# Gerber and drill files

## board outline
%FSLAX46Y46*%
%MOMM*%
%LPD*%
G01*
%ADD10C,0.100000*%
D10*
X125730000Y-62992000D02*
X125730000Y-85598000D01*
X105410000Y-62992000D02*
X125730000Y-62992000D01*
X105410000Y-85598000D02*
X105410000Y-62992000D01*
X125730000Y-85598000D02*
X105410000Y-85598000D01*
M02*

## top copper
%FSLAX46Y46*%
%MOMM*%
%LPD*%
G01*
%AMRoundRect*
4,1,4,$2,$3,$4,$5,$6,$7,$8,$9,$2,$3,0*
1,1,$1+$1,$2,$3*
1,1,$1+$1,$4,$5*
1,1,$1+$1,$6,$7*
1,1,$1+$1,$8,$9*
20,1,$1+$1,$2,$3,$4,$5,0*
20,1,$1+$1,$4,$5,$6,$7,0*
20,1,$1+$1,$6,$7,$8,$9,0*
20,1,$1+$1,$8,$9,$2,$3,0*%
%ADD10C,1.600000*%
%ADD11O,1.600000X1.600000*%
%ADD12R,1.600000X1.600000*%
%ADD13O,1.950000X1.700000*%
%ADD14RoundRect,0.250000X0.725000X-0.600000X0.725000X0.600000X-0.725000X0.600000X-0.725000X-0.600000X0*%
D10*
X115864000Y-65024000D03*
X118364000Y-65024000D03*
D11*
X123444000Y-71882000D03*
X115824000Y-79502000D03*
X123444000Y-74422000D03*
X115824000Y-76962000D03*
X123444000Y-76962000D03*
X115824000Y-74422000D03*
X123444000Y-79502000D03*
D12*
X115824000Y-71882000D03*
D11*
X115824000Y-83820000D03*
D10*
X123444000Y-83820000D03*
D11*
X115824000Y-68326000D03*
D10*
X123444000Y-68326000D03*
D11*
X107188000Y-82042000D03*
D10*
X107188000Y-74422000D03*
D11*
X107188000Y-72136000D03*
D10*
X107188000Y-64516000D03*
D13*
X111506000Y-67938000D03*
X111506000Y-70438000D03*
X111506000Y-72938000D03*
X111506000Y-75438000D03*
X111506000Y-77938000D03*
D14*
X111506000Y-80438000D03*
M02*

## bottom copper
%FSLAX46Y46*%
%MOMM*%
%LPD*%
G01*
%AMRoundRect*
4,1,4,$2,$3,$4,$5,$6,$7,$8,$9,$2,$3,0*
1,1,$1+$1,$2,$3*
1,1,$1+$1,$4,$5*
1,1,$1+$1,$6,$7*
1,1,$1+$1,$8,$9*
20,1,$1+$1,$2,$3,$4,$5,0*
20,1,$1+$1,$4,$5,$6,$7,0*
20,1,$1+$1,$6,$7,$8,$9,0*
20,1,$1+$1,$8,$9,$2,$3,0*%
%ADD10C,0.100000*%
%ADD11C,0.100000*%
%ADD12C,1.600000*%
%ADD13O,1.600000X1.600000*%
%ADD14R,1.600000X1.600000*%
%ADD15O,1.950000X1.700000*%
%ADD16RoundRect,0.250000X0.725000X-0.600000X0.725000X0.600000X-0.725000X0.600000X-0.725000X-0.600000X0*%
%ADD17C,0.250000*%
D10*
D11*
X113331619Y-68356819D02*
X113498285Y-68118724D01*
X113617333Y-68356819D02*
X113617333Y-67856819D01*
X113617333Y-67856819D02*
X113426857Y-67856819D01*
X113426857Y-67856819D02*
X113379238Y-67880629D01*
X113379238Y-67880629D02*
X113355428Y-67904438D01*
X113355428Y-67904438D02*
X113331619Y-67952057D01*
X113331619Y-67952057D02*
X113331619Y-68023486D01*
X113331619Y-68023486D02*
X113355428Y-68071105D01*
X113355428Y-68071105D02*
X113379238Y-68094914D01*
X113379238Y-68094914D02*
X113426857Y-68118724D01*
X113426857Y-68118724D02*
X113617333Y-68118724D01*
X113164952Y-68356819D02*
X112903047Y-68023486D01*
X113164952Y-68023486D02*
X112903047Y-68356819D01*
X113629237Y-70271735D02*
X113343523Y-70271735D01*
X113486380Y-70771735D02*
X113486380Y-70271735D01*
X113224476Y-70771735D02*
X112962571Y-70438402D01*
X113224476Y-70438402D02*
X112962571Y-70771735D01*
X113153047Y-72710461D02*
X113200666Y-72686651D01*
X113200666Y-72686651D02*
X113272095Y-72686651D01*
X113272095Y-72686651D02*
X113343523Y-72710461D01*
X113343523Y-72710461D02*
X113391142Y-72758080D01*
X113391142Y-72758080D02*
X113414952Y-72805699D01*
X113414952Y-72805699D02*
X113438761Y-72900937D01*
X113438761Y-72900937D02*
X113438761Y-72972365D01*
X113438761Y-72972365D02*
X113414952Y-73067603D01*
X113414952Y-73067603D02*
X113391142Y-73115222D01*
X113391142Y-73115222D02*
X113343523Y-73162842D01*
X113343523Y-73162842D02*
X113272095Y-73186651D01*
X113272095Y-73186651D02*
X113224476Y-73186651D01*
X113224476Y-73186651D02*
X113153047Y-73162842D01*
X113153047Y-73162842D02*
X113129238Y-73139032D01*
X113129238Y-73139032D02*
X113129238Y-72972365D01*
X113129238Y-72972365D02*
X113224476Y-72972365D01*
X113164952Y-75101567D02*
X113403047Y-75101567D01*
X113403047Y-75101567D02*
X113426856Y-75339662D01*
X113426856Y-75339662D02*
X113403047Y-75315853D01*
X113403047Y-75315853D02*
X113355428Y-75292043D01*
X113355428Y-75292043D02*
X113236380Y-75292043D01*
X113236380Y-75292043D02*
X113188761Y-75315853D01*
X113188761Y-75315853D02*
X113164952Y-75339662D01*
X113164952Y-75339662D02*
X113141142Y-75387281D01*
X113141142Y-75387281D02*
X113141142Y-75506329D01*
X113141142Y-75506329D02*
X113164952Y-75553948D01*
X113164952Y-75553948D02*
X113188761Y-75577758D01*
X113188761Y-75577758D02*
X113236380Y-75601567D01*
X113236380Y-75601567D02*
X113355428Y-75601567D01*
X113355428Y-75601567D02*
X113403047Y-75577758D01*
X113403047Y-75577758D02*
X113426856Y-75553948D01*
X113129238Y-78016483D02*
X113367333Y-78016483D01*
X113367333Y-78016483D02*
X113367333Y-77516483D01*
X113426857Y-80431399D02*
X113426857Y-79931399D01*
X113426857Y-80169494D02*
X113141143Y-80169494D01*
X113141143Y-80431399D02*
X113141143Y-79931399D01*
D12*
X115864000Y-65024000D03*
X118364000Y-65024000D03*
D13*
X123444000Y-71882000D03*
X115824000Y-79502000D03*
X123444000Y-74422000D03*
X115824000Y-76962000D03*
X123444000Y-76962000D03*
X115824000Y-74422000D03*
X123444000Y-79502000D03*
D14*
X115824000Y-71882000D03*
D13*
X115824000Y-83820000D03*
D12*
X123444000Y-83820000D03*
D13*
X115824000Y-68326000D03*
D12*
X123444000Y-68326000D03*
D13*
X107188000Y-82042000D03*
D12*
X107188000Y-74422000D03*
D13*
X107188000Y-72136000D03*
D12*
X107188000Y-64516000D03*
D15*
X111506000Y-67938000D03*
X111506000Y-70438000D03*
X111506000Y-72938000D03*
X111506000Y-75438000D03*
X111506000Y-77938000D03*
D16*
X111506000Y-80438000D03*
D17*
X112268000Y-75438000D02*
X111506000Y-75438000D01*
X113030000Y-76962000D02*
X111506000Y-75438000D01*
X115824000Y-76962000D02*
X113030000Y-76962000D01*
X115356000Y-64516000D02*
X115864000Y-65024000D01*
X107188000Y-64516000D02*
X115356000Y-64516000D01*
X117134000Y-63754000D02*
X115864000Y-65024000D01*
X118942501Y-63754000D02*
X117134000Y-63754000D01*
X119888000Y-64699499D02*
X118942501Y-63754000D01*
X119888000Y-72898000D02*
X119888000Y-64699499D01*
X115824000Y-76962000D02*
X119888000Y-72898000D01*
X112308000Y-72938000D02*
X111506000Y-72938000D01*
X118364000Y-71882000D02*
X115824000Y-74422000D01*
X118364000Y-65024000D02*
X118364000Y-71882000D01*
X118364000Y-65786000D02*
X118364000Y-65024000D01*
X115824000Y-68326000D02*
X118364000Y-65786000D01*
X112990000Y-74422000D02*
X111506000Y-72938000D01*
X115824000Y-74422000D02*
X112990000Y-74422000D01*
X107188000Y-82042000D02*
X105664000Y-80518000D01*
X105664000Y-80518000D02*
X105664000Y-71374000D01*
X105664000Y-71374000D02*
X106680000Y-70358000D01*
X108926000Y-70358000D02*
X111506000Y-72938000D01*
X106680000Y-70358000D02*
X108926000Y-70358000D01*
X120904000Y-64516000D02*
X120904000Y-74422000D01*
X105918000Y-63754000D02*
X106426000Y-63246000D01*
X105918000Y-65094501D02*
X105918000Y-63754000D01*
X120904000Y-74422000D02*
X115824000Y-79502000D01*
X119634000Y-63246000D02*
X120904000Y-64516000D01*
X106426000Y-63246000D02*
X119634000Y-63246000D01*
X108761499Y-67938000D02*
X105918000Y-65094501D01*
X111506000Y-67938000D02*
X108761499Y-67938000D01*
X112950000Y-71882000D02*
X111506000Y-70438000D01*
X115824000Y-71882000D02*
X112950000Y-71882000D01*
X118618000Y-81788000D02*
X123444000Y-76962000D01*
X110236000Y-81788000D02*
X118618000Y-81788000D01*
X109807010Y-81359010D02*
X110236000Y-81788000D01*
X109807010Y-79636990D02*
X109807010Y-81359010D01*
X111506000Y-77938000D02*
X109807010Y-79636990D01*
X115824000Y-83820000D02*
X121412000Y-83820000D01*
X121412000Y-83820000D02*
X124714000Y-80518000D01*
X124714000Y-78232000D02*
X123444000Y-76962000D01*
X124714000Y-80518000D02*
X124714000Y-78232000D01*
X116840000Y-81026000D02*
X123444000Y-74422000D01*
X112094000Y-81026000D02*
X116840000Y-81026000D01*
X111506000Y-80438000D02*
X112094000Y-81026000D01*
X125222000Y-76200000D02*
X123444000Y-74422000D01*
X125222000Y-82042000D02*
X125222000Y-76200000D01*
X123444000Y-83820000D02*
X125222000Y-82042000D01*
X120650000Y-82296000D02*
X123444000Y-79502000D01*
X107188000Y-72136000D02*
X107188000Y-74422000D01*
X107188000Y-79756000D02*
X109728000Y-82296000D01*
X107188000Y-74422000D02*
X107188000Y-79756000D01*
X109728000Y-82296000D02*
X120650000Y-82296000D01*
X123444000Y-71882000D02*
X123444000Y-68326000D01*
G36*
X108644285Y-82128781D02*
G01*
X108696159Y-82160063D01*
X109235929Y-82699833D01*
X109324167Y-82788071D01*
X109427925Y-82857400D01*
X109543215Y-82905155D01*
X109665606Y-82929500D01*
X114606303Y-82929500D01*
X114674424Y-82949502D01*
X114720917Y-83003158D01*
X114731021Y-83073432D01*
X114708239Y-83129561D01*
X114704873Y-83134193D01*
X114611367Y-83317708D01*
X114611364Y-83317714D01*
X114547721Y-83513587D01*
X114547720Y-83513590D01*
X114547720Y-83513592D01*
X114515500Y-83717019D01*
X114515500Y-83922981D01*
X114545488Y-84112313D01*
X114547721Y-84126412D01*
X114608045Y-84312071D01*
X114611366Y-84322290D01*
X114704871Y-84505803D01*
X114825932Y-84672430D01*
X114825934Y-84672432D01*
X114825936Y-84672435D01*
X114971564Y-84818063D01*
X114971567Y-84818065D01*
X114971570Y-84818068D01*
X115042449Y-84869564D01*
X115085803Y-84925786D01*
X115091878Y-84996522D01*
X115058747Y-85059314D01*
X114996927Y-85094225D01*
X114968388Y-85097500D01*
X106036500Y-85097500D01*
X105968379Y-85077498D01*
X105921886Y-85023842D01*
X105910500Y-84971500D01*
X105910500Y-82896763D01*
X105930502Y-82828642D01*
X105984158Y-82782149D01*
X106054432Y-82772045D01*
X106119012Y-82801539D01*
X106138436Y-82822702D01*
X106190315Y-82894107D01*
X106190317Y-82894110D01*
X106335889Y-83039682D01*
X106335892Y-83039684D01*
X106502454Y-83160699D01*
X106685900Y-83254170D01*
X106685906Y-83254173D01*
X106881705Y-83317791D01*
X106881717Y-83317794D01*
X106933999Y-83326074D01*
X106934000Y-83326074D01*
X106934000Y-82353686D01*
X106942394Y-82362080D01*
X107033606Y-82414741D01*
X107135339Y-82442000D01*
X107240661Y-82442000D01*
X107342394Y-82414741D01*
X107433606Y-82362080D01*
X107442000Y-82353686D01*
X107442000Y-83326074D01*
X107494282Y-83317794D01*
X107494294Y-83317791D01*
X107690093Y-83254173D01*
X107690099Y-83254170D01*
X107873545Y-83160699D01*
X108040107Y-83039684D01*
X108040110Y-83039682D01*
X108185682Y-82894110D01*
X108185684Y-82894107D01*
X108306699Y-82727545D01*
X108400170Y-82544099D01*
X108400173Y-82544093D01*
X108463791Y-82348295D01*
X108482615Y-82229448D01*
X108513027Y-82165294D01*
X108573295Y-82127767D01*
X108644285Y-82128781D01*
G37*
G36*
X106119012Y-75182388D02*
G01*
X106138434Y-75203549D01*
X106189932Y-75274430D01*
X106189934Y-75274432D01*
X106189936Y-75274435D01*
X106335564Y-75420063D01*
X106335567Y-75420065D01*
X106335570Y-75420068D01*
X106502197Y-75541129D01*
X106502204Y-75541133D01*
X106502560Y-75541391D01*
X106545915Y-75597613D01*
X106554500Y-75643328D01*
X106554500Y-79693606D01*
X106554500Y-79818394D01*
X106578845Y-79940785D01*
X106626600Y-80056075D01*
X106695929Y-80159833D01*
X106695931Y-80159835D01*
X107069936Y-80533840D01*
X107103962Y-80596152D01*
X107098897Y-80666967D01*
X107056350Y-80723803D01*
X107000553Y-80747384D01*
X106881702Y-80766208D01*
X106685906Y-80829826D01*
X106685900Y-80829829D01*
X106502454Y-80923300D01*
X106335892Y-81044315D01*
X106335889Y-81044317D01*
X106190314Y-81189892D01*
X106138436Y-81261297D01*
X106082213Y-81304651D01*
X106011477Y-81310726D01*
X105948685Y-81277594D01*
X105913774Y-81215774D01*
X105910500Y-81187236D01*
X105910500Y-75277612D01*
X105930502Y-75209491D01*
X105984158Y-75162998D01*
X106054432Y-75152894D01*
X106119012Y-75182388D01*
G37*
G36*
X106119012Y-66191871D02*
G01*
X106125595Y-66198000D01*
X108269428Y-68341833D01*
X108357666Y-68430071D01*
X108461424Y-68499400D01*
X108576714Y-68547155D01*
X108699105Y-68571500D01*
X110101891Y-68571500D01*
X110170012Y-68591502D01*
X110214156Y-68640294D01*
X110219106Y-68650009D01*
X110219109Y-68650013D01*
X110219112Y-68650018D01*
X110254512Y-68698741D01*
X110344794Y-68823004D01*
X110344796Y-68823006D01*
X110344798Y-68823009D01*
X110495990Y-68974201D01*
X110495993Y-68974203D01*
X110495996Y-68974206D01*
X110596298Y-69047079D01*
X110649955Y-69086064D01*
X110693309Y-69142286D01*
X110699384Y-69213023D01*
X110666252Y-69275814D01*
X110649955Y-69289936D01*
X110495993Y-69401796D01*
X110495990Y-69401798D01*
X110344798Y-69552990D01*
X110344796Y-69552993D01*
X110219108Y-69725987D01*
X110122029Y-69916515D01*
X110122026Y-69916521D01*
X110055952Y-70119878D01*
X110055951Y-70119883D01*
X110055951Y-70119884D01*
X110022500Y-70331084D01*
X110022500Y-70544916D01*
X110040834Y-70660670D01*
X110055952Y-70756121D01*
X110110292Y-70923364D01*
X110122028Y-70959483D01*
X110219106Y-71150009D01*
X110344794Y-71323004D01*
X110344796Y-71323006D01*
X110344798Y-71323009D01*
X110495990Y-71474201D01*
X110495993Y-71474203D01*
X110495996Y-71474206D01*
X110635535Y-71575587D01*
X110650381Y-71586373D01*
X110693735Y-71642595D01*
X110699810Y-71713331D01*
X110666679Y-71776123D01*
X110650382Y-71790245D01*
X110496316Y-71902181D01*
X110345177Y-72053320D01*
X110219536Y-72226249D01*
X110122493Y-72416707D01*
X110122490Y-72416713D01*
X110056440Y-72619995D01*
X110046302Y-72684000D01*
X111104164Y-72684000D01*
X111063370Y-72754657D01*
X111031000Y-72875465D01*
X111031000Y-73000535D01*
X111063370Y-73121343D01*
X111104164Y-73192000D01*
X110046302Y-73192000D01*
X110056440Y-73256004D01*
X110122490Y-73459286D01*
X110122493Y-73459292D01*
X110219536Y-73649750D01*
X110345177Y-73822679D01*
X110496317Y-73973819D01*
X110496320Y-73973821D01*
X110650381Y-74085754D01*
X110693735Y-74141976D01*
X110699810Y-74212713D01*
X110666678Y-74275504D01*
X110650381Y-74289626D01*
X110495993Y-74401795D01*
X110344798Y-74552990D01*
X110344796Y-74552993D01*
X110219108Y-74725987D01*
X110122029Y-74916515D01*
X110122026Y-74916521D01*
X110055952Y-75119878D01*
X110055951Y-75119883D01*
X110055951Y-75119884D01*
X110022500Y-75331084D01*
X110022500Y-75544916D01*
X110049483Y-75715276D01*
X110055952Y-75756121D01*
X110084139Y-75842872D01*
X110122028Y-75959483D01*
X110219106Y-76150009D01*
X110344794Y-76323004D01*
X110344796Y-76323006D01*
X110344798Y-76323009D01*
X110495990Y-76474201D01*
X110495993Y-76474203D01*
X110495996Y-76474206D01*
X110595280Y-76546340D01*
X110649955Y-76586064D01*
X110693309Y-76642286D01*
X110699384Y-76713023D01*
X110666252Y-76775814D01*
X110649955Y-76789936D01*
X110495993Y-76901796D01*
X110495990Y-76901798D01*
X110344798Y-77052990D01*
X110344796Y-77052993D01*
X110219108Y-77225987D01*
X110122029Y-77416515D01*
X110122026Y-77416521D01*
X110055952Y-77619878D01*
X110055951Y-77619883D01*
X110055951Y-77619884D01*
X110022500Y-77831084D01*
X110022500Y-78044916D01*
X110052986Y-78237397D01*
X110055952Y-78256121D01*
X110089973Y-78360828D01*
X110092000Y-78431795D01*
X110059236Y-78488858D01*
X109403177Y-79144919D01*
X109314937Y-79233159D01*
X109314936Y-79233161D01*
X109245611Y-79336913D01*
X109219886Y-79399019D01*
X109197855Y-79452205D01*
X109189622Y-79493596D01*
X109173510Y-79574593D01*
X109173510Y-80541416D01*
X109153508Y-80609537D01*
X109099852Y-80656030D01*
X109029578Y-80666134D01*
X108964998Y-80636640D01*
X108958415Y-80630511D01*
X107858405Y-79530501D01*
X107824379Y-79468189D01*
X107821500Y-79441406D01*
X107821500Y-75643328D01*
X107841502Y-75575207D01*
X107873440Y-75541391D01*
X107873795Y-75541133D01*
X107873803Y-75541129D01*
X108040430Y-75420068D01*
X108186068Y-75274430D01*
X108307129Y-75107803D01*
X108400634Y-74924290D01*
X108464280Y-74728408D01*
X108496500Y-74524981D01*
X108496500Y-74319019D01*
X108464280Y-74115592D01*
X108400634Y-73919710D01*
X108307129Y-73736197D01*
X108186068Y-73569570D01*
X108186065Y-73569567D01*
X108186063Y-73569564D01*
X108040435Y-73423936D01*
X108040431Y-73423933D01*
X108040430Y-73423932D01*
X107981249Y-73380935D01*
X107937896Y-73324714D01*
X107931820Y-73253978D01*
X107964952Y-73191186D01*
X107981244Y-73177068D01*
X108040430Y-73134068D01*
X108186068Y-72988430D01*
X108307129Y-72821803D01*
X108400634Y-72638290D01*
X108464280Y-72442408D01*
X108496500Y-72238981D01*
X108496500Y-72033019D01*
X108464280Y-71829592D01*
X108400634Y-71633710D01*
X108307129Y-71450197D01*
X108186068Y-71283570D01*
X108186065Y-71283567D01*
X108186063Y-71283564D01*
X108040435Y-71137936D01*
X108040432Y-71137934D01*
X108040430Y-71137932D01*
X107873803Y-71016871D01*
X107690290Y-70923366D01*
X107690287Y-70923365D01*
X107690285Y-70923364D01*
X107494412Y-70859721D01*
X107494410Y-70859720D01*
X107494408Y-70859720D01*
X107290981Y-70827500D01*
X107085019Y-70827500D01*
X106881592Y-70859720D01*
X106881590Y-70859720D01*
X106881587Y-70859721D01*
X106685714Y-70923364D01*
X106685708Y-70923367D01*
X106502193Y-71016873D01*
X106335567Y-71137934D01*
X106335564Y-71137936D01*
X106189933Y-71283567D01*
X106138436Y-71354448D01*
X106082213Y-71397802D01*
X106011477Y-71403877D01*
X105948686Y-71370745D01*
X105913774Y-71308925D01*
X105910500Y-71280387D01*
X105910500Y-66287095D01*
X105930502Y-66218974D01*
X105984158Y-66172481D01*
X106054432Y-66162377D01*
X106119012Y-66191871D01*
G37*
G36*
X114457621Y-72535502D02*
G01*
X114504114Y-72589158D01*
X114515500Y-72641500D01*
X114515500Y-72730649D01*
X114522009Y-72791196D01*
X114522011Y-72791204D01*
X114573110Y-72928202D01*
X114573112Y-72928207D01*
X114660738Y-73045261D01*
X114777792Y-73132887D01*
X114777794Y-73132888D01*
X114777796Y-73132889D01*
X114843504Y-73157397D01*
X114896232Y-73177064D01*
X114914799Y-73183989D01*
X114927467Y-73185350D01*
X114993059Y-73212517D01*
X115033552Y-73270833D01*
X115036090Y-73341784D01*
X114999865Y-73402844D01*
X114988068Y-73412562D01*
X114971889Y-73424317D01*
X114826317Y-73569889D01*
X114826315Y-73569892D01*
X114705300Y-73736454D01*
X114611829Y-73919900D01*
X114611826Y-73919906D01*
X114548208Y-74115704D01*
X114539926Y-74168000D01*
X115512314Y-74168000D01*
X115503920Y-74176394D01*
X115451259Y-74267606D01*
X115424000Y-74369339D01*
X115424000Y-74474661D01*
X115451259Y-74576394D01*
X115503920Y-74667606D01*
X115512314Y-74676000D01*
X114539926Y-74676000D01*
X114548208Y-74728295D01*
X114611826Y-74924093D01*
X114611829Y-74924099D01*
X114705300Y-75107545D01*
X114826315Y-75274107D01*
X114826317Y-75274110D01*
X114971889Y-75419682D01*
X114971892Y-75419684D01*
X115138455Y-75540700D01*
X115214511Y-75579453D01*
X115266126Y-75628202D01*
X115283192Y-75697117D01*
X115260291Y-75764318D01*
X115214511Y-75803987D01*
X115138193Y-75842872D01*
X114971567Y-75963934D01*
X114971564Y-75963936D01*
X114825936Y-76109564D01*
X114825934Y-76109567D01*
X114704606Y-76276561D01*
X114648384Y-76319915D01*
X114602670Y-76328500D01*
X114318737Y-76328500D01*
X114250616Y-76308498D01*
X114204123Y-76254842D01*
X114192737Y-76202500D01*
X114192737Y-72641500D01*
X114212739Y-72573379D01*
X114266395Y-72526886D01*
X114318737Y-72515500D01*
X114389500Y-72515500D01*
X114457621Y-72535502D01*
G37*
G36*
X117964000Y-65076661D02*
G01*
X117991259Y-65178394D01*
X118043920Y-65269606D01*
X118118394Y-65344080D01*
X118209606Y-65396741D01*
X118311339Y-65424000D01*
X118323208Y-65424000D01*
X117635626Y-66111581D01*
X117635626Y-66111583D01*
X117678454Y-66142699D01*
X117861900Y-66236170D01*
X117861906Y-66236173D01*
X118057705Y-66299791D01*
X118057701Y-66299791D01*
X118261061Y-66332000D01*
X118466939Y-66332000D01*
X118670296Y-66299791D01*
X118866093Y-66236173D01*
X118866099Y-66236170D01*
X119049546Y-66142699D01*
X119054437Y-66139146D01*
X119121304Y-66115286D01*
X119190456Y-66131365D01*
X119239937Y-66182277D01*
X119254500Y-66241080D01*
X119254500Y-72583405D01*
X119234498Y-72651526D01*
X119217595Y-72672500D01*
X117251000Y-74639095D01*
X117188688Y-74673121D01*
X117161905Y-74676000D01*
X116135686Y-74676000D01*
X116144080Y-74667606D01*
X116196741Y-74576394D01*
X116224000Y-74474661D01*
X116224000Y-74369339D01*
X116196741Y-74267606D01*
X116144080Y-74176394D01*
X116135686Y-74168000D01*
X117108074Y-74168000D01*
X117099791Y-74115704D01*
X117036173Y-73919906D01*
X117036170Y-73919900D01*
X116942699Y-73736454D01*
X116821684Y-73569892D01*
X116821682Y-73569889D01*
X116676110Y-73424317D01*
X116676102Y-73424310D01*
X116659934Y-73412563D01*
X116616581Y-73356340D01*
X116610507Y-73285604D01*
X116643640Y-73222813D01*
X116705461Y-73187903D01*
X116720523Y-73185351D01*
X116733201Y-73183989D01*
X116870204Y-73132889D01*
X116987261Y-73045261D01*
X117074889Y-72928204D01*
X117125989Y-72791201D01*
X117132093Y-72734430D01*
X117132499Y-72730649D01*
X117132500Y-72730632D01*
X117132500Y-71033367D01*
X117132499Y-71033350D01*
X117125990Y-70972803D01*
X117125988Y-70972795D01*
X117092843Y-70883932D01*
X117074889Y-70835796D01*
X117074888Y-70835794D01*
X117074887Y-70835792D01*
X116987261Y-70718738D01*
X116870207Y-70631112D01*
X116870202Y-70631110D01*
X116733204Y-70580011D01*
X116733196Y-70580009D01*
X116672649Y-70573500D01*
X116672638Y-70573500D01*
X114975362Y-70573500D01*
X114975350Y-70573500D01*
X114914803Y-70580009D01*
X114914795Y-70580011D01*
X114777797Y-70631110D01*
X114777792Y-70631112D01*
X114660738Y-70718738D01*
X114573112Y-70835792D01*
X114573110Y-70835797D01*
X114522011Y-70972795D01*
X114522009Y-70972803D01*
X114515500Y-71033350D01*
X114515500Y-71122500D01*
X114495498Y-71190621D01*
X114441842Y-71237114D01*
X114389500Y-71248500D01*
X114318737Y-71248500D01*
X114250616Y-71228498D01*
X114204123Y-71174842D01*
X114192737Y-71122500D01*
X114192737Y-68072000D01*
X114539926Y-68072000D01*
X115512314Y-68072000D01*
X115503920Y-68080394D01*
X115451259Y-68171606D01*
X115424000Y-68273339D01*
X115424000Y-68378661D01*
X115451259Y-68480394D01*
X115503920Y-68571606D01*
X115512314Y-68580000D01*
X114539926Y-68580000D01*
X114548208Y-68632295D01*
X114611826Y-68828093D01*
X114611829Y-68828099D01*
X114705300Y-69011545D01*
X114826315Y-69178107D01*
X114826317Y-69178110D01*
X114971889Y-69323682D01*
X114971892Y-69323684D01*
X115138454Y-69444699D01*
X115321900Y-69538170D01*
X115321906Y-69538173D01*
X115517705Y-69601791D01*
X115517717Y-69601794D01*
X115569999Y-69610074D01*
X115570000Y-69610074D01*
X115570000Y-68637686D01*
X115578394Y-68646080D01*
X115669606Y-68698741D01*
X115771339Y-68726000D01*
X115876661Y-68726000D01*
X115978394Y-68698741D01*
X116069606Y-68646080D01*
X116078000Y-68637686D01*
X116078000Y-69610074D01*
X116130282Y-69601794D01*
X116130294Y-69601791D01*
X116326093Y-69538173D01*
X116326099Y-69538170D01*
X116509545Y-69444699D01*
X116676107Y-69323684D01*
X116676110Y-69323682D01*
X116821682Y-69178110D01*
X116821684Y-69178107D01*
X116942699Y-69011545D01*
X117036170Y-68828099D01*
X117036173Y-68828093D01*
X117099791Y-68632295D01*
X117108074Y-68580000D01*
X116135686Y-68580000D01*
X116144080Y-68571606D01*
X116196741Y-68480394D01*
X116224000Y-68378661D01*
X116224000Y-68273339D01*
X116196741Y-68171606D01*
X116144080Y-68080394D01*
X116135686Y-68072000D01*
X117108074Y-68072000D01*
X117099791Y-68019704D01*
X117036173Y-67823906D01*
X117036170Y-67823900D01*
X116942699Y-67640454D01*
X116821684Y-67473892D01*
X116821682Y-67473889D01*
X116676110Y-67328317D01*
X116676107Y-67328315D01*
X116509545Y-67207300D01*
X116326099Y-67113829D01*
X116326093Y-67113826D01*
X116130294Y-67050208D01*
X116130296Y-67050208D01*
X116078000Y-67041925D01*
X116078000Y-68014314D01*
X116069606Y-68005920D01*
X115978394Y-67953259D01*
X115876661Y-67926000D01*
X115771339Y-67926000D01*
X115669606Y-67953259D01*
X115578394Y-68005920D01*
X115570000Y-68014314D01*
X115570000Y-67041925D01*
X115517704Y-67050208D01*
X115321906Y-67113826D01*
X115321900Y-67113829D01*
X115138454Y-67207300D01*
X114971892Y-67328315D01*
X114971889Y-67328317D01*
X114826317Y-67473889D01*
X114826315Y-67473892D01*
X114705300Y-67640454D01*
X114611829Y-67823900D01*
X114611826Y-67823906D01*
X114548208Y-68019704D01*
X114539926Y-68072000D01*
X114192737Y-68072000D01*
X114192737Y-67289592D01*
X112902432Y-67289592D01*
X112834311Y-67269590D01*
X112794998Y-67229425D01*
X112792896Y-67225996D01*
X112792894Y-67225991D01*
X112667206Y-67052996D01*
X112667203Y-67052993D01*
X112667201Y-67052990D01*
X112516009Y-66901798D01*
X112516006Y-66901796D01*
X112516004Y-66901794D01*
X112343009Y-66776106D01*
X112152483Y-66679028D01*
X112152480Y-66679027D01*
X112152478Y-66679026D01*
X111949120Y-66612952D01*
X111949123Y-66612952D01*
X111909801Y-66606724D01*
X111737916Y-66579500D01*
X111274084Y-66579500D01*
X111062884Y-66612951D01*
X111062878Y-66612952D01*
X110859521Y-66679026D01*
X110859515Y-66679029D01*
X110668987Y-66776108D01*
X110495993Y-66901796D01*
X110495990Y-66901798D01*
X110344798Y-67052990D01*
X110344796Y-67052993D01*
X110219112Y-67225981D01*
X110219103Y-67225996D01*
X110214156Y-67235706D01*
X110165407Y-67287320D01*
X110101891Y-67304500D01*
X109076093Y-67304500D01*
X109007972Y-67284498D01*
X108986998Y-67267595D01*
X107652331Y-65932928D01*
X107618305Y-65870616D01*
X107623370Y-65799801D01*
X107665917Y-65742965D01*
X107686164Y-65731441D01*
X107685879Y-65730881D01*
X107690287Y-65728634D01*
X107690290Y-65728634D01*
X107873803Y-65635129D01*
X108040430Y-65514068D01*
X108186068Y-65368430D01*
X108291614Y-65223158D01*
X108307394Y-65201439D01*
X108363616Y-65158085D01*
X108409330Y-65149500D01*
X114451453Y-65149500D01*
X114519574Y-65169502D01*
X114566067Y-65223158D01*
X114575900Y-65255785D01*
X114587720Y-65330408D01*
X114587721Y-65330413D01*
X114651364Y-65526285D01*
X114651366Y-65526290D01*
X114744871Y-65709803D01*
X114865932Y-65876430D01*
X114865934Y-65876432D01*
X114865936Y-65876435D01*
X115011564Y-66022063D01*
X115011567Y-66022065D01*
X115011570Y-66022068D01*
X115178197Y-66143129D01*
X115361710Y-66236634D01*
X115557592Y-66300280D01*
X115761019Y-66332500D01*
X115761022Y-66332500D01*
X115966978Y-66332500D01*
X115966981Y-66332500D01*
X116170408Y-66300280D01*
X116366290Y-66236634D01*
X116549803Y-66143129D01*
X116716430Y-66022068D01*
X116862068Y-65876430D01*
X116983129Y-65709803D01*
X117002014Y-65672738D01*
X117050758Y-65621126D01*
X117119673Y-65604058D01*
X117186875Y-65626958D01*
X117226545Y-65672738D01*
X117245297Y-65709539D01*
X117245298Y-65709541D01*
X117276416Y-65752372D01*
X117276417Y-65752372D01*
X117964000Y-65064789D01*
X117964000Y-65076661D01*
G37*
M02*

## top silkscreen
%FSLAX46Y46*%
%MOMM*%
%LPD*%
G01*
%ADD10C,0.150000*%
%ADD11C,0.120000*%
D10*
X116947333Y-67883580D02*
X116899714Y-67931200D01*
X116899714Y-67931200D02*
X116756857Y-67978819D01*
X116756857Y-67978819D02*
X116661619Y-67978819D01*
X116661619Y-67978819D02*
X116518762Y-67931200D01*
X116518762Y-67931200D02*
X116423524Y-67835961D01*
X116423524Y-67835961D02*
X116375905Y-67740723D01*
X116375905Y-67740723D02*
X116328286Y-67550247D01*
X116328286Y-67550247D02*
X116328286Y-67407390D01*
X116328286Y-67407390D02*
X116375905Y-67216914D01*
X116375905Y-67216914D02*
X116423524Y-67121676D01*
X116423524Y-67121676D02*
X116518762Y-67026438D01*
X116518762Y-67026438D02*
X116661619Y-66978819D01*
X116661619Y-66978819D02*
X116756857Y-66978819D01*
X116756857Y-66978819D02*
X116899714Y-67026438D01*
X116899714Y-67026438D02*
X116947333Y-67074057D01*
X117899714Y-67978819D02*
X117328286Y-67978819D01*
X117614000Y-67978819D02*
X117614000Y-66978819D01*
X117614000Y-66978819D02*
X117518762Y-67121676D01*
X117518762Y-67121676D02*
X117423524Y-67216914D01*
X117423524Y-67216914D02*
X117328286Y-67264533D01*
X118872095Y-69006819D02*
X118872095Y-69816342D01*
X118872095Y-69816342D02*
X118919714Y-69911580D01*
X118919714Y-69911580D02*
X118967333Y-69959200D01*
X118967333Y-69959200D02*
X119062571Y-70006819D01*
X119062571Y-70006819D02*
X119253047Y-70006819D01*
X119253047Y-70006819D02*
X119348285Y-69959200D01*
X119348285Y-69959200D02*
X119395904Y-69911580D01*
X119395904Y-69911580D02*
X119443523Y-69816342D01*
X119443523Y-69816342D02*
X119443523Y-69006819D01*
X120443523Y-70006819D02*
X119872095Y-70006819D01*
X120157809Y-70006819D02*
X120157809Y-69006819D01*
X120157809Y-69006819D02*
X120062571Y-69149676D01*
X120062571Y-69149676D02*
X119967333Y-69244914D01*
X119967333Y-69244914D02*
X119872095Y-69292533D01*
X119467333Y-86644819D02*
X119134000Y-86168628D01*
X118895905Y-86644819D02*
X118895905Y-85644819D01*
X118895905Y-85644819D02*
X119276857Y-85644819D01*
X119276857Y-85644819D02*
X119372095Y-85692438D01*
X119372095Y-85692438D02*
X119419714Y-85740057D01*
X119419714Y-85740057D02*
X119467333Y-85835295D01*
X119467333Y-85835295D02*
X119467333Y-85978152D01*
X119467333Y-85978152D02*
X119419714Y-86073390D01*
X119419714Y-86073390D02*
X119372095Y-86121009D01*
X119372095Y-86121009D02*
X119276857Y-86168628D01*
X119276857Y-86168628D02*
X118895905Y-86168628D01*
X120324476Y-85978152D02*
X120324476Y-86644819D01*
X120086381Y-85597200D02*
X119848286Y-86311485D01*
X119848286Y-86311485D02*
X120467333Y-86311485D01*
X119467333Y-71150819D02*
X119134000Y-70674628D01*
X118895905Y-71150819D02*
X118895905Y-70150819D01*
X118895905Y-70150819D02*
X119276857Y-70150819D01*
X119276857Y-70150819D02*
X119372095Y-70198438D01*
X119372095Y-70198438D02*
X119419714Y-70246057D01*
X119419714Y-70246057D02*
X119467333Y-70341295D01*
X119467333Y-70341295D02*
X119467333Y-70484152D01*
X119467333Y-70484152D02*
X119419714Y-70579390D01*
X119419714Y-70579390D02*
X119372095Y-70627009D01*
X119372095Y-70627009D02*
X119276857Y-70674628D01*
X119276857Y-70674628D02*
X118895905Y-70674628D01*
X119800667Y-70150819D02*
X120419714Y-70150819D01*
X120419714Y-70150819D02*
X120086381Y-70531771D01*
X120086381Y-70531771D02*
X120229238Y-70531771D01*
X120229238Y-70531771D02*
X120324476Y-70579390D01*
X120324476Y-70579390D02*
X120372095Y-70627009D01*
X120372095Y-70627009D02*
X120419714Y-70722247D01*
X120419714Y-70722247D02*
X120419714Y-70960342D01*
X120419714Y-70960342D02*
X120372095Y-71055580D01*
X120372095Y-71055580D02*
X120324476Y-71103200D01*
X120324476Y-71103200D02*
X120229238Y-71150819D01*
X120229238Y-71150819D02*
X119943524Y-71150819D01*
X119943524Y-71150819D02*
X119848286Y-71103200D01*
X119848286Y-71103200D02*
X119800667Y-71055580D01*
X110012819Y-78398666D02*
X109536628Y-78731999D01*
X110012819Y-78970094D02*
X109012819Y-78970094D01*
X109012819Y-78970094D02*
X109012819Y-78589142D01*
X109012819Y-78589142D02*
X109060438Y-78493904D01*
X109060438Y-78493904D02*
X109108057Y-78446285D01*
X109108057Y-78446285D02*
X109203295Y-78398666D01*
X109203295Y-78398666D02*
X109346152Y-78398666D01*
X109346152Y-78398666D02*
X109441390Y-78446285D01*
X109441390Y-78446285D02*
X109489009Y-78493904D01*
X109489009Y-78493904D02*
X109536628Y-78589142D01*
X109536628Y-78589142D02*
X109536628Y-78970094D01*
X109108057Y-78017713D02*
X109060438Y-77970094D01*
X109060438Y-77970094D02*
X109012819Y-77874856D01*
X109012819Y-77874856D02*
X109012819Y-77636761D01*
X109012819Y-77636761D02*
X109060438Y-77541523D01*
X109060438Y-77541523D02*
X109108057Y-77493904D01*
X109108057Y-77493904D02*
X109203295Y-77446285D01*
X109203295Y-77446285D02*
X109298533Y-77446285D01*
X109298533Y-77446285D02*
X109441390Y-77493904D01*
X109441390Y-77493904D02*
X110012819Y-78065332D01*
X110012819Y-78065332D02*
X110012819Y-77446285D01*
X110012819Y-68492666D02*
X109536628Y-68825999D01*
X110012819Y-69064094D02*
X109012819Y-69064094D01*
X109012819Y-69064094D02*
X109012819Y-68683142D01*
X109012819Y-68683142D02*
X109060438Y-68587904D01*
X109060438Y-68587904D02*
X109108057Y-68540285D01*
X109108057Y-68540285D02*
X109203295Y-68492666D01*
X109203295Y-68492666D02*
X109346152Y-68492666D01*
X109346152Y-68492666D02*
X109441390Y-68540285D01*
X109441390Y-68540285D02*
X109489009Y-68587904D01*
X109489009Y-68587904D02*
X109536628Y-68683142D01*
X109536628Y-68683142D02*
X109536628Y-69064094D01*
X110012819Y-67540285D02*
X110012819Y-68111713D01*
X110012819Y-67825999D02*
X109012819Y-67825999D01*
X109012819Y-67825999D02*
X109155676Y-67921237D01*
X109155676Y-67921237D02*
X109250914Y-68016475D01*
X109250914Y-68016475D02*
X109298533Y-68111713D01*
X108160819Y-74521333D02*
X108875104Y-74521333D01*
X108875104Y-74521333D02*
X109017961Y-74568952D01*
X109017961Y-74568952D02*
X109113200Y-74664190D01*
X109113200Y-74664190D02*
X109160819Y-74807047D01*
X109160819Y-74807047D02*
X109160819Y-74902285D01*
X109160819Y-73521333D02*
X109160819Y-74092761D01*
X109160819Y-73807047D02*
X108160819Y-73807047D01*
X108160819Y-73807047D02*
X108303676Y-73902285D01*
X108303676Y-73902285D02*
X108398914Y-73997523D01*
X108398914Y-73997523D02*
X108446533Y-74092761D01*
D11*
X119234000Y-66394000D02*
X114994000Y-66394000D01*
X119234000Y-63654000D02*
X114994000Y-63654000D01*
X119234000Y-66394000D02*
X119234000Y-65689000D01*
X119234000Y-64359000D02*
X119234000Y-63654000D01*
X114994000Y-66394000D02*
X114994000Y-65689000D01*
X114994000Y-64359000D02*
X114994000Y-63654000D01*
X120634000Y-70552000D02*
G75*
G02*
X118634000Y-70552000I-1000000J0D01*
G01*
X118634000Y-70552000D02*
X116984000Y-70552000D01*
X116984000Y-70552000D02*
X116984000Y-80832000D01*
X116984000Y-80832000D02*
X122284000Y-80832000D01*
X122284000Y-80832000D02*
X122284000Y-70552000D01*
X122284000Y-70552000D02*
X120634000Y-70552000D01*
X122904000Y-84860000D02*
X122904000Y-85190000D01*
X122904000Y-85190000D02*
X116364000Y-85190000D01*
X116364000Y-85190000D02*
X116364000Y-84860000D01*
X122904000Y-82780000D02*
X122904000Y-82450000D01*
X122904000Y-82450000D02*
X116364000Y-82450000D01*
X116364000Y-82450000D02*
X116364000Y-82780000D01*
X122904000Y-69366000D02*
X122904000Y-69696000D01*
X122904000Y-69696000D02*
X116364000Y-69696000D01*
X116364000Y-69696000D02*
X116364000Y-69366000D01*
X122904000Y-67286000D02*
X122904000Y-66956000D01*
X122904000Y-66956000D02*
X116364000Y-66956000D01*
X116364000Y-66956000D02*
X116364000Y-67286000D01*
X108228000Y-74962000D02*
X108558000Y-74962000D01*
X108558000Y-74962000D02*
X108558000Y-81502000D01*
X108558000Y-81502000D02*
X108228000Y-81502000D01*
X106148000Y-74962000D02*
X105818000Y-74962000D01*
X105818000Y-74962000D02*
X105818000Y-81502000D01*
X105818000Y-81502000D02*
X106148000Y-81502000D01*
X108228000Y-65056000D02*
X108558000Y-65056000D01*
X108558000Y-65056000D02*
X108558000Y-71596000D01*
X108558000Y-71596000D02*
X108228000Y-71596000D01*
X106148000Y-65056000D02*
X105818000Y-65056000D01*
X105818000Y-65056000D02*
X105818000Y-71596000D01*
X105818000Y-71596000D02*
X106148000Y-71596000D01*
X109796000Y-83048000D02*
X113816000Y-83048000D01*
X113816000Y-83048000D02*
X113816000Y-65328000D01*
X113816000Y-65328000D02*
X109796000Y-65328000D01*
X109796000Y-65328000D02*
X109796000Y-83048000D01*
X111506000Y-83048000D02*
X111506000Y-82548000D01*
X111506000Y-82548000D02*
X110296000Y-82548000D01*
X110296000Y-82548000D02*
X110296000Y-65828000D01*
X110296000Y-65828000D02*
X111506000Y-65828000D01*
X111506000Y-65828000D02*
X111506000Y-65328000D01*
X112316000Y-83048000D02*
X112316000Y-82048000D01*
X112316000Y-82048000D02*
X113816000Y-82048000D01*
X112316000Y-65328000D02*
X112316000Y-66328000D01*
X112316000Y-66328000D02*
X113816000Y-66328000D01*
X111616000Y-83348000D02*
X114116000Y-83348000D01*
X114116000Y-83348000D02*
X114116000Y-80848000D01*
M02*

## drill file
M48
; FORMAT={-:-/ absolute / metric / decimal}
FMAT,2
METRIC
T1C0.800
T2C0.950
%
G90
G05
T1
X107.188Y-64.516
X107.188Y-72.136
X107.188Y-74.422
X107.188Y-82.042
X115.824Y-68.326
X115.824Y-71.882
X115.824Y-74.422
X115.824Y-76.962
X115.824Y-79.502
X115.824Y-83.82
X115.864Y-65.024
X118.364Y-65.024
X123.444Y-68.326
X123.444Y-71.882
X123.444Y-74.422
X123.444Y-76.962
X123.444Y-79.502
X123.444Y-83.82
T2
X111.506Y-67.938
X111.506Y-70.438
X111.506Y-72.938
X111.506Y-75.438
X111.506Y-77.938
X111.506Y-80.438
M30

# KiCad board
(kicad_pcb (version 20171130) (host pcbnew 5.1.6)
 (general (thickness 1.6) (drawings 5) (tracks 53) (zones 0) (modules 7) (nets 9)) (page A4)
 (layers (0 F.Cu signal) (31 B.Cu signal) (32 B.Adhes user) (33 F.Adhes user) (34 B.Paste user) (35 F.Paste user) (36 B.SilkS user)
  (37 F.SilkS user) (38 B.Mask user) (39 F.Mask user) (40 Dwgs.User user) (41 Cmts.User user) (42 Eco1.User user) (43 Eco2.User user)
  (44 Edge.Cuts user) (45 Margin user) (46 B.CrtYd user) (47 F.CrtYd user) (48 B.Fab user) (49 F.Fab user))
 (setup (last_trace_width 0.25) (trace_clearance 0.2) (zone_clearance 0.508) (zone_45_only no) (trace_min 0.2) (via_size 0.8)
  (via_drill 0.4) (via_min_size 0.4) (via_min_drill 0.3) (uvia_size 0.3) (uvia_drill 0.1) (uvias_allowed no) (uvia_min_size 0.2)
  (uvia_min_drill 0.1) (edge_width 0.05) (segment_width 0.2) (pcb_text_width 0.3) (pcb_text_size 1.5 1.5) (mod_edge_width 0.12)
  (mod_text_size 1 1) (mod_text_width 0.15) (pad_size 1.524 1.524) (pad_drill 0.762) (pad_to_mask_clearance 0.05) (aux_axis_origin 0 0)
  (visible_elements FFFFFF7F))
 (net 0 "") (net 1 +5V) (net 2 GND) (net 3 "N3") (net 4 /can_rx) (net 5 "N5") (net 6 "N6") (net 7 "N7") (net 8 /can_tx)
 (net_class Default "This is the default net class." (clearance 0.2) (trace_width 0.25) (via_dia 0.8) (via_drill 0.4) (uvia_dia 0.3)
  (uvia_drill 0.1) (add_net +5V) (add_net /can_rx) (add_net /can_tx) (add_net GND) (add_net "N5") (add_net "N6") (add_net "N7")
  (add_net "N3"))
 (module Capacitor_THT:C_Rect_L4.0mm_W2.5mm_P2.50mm (layer F.Cu) (at 118.364 65.024 180)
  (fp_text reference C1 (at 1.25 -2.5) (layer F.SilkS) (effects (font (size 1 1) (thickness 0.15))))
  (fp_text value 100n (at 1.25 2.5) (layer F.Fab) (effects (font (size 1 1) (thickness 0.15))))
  (fp_line (start -0.87 -1.37) (end 3.37 -1.37) (layer F.SilkS) (width 0.12))
  (fp_line (start -0.87 1.37) (end 3.37 1.37) (layer F.SilkS) (width 0.12))
  (fp_line (start -0.87 -1.37) (end -0.87 -0.665) (layer F.SilkS) (width 0.12))
  (fp_line (start -0.87 0.665) (end -0.87 1.37) (layer F.SilkS) (width 0.12))
  (fp_line (start 3.37 -1.37) (end 3.37 -0.665) (layer F.SilkS) (width 0.12))
  (fp_line (start 3.37 0.665) (end 3.37 1.37) (layer F.SilkS) (width 0.12))
  (pad 2 thru_hole circle (at 2.5 0 180) (size 1.6 1.6) (drill 0.8) (layers *.Cu *.Mask) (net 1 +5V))
  (pad 1 thru_hole circle (at 0 0 180) (size 1.6 1.6) (drill 0.8) (layers *.Cu *.Mask) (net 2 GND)))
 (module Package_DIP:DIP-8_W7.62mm (layer F.Cu) (at 115.824 71.882)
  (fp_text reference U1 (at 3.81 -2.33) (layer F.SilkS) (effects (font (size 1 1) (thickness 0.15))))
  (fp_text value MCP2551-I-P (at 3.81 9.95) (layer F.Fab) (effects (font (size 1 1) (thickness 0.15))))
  (fp_arc (start 3.81 -1.33) (end 2.81 -1.33) (angle -180) (layer F.SilkS) (width 0.12))
  (fp_line (start 2.81 -1.33) (end 1.16 -1.33) (layer F.SilkS) (width 0.12))
  (fp_line (start 1.16 -1.33) (end 1.16 8.95) (layer F.SilkS) (width 0.12))
  (fp_line (start 1.16 8.95) (end 6.46 8.95) (layer F.SilkS) (width 0.12))
  (fp_line (start 6.46 8.95) (end 6.46 -1.33) (layer F.SilkS) (width 0.12))
  (fp_line (start 6.46 -1.33) (end 4.81 -1.33) (layer F.SilkS) (width 0.12))
  (pad 8 thru_hole oval (at 7.62 0) (size 1.6 1.6) (drill 0.8) (layers *.Cu *.Mask) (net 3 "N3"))
  (pad 4 thru_hole oval (at 0 7.62) (size 1.6 1.6) (drill 0.8) (layers *.Cu *.Mask) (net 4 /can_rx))
  (pad 7 thru_hole oval (at 7.62 2.54) (size 1.6 1.6) (drill 0.8) (layers *.Cu *.Mask) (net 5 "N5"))
  (pad 3 thru_hole oval (at 0 5.08) (size 1.6 1.6) (drill 0.8) (layers *.Cu *.Mask) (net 1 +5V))
  (pad 6 thru_hole oval (at 7.62 5.08) (size 1.6 1.6) (drill 0.8) (layers *.Cu *.Mask) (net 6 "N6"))
  (pad 2 thru_hole oval (at 0 2.54) (size 1.6 1.6) (drill 0.8) (layers *.Cu *.Mask) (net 2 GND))
  (pad 5 thru_hole oval (at 7.62 7.62) (size 1.6 1.6) (drill 0.8) (layers *.Cu *.Mask) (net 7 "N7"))
  (pad 1 thru_hole rect (at 0 0) (size 1.6 1.6) (drill 0.8) (layers *.Cu *.Mask) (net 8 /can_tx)))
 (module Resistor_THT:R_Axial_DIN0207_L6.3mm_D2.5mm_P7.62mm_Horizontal (layer F.Cu) (at 123.444 83.82 180)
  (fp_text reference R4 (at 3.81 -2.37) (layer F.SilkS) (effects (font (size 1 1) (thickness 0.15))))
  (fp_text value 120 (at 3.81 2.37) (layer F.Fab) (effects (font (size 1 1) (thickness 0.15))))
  (fp_line (start 0.54 -1.04) (end 0.54 -1.37) (layer F.SilkS) (width 0.12))
  (fp_line (start 0.54 -1.37) (end 7.08 -1.37) (layer F.SilkS) (width 0.12))
  (fp_line (start 7.08 -1.37) (end 7.08 -1.04) (layer F.SilkS) (width 0.12))
  (fp_line (start 0.54 1.04) (end 0.54 1.37) (layer F.SilkS) (width 0.12))
  (fp_line (start 0.54 1.37) (end 7.08 1.37) (layer F.SilkS) (width 0.12))
  (fp_line (start 7.08 1.37) (end 7.08 1.04) (layer F.SilkS) (width 0.12))
  (pad 2 thru_hole oval (at 7.62 0 180) (size 1.6 1.6) (drill 0.8) (layers *.Cu *.Mask) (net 6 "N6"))
  (pad 1 thru_hole circle (at 0 0 180) (size 1.6 1.6) (drill 0.8) (layers *.Cu *.Mask) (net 5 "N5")))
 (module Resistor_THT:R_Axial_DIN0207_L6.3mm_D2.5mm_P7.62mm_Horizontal (layer F.Cu) (at 123.444 68.326 180)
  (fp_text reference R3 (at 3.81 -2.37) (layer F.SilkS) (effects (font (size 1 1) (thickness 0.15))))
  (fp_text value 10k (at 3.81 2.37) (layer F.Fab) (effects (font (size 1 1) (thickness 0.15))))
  (fp_line (start 0.54 -1.04) (end 0.54 -1.37) (layer F.SilkS) (width 0.12))
  (fp_line (start 0.54 -1.37) (end 7.08 -1.37) (layer F.SilkS) (width 0.12))
  (fp_line (start 7.08 -1.37) (end 7.08 -1.04) (layer F.SilkS) (width 0.12))
  (fp_line (start 0.54 1.04) (end 0.54 1.37) (layer F.SilkS) (width 0.12))
  (fp_line (start 0.54 1.37) (end 7.08 1.37) (layer F.SilkS) (width 0.12))
  (fp_line (start 7.08 1.37) (end 7.08 1.04) (layer F.SilkS) (width 0.12))
  (pad 2 thru_hole oval (at 7.62 0 180) (size 1.6 1.6) (drill 0.8) (layers *.Cu *.Mask) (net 2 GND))
  (pad 1 thru_hole circle (at 0 0 180) (size 1.6 1.6) (drill 0.8) (layers *.Cu *.Mask) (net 3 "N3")))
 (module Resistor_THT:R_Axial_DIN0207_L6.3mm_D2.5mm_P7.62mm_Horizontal (layer F.Cu) (at 107.188 74.422 270)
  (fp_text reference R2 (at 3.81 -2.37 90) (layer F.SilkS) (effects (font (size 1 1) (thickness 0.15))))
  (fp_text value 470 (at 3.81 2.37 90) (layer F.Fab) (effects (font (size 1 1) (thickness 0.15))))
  (fp_line (start 0.54 -1.04) (end 0.54 -1.37) (layer F.SilkS) (width 0.12))
  (fp_line (start 0.54 -1.37) (end 7.08 -1.37) (layer F.SilkS) (width 0.12))
  (fp_line (start 7.08 -1.37) (end 7.08 -1.04) (layer F.SilkS) (width 0.12))
  (fp_line (start 0.54 1.04) (end 0.54 1.37) (layer F.SilkS) (width 0.12))
  (fp_line (start 0.54 1.37) (end 7.08 1.37) (layer F.SilkS) (width 0.12))
  (fp_line (start 7.08 1.37) (end 7.08 1.04) (layer F.SilkS) (width 0.12))
  (pad 2 thru_hole oval (at 7.62 0 270) (size 1.6 1.6) (drill 0.8) (layers *.Cu *.Mask) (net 2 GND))
  (pad 1 thru_hole circle (at 0 0 270) (size 1.6 1.6) (drill 0.8) (layers *.Cu *.Mask) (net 7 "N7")))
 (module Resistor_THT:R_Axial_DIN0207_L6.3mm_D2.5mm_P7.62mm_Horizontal (layer F.Cu) (at 107.188 64.516 270)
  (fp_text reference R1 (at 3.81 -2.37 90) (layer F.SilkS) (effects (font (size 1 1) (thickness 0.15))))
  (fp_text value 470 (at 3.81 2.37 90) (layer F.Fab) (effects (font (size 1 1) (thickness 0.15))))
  (fp_line (start 0.54 -1.04) (end 0.54 -1.37) (layer F.SilkS) (width 0.12))
  (fp_line (start 0.54 -1.37) (end 7.08 -1.37) (layer F.SilkS) (width 0.12))
  (fp_line (start 7.08 -1.37) (end 7.08 -1.04) (layer F.SilkS) (width 0.12))
  (fp_line (start 0.54 1.04) (end 0.54 1.37) (layer F.SilkS) (width 0.12))
  (fp_line (start 0.54 1.37) (end 7.08 1.37) (layer F.SilkS) (width 0.12))
  (fp_line (start 7.08 1.37) (end 7.08 1.04) (layer F.SilkS) (width 0.12))
  (pad 2 thru_hole oval (at 7.62 0 270) (size 1.6 1.6) (drill 0.8) (layers *.Cu *.Mask) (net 7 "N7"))
  (pad 1 thru_hole circle (at 0 0 270) (size 1.6 1.6) (drill 0.8) (layers *.Cu *.Mask) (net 1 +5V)))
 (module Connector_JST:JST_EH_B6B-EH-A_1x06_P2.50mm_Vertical (layer F.Cu) (at 111.506 80.438 90)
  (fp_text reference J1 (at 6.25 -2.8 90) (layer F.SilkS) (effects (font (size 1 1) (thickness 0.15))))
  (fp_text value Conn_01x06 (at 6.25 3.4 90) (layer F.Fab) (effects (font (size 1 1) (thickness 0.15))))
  (fp_line (start -2.61 -1.71) (end -2.61 2.31) (layer F.SilkS) (width 0.12))
  (fp_line (start -2.61 2.31) (end 15.11 2.31) (layer F.SilkS) (width 0.12))
  (fp_line (start 15.11 2.31) (end 15.11 -1.71) (layer F.SilkS) (width 0.12))
  (fp_line (start 15.11 -1.71) (end -2.61 -1.71) (layer F.SilkS) (width 0.12))
  (fp_line (start -2.61 0) (end -2.11 0) (layer F.SilkS) (width 0.12))
  (fp_line (start -2.11 0) (end -2.11 -1.21) (layer F.SilkS) (width 0.12))
  (fp_line (start -2.11 -1.21) (end 14.61 -1.21) (layer F.SilkS) (width 0.12))
  (fp_line (start 14.61 -1.21) (end 14.61 0) (layer F.SilkS) (width 0.12))
  (fp_line (start 14.61 0) (end 15.11 0) (layer F.SilkS) (width 0.12))
  (fp_line (start -2.61 0.81) (end -1.61 0.81) (layer F.SilkS) (width 0.12))
  (fp_line (start -1.61 0.81) (end -1.61 2.31) (layer F.SilkS) (width 0.12))
  (fp_line (start 15.11 0.81) (end 14.11 0.81) (layer F.SilkS) (width 0.12))
  (fp_line (start 14.11 0.81) (end 14.11 2.31) (layer F.SilkS) (width 0.12))
  (fp_line (start -2.91 0.11) (end -2.91 2.61) (layer F.SilkS) (width 0.12))
  (fp_line (start -2.91 2.61) (end -0.41 2.61) (layer F.SilkS) (width 0.12))
  (pad 6 thru_hole oval (at 12.5 0 90) (size 1.7 1.95) (drill 0.95) (layers *.Cu *.Mask) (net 4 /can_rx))
  (pad 5 thru_hole oval (at 10 0 90) (size 1.7 1.95) (drill 0.95) (layers *.Cu *.Mask) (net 8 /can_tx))
  (pad 4 thru_hole oval (at 7.5 0 90) (size 1.7 1.95) (drill 0.95) (layers *.Cu *.Mask) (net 2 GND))
  (pad 3 thru_hole oval (at 5 0 90) (size 1.7 1.95) (drill 0.95) (layers *.Cu *.Mask) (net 1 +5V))
  (pad 2 thru_hole oval (at 2.5 0 90) (size 1.7 1.95) (drill 0.95) (layers *.Cu *.Mask) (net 6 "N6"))
  (pad 1 thru_hole roundrect (at 0 0 90) (size 1.7 1.95) (drill 0.95) (layers *.Cu *.Mask) (roundrect_rratio 0.147059) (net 5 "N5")))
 (gr_line (start 125.73 62.992) (end 125.73 85.598) (layer Edge.Cuts) (width 0.1))
 (gr_line (start 105.41 62.992) (end 125.73 62.992) (layer Edge.Cuts) (width 0.1))
 (gr_line (start 105.41 85.598) (end 105.41 62.992) (layer Edge.Cuts) (width 0.1))
 (gr_line (start 125.73 85.598) (end 105.41 85.598) (layer Edge.Cuts) (width 0.1))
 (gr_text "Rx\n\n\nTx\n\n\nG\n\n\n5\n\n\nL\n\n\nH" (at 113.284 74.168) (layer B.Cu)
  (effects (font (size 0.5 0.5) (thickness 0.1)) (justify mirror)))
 (segment (start 112.268 75.438) (end 111.506 75.438) (width 0.25) (layer B.Cu) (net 1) (status 30))
 (segment (start 113.03 76.962) (end 111.506 75.438) (width 0.25) (layer B.Cu) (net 1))
 (segment (start 115.824 76.962) (end 113.03 76.962) (width 0.25) (layer B.Cu) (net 1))
 (segment (start 115.356 64.516) (end 115.864 65.024) (width 0.25) (layer B.Cu) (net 1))
 (segment (start 107.188 64.516) (end 115.356 64.516) (width 0.25) (layer B.Cu) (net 1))
 (segment (start 117.134 63.754) (end 115.864 65.024) (width 0.25) (layer B.Cu) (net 1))
 (segment (start 118.942501 63.754) (end 117.134 63.754) (width 0.25) (layer B.Cu) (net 1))
 (segment (start 119.888 64.699499) (end 118.942501 63.754) (width 0.25) (layer B.Cu) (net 1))
 (segment (start 119.888 72.898) (end 119.888 64.699499) (width 0.25) (layer B.Cu) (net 1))
 (segment (start 115.824 76.962) (end 119.888 72.898) (width 0.25) (layer B.Cu) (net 1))
 (segment (start 112.308 72.938) (end 111.506 72.938) (width 0.25) (layer B.Cu) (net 2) (status 30))
 (segment (start 118.364 71.882) (end 115.824 74.422) (width 0.25) (layer B.Cu) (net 2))
 (segment (start 118.364 65.024) (end 118.364 71.882) (width 0.25) (layer B.Cu) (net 2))
 (segment (start 118.364 65.786) (end 118.364 65.024) (width 0.25) (layer B.Cu) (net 2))
 (segment (start 115.824 68.326) (end 118.364 65.786) (width 0.25) (layer B.Cu) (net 2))
 (segment (start 112.99 74.422) (end 111.506 72.938) (width 0.25) (layer B.Cu) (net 2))
 (segment (start 115.824 74.422) (end 112.99 74.422) (width 0.25) (layer B.Cu) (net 2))
 (segment (start 107.188 82.042) (end 105.664 80.518) (width 0.25) (layer B.Cu) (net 2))
 (segment (start 105.664 80.518) (end 105.664 71.374) (width 0.25) (layer B.Cu) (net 2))
 (segment (start 105.664 71.374) (end 106.68 70.358) (width 0.25) (layer B.Cu) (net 2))
 (segment (start 108.926 70.358) (end 111.506 72.938) (width 0.25) (layer B.Cu) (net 2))
 (segment (start 106.68 70.358) (end 108.926 70.358) (width 0.25) (layer B.Cu) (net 2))
 (segment (start 120.904 64.516) (end 120.904 74.422) (width 0.25) (layer B.Cu) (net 4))
 (segment (start 105.918 63.754) (end 106.426 63.246) (width 0.25) (layer B.Cu) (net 4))
 (segment (start 105.918 65.094501) (end 105.918 63.754) (width 0.25) (layer B.Cu) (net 4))
 (segment (start 120.904 74.422) (end 115.824 79.502) (width 0.25) (layer B.Cu) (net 4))
 (segment (start 119.634 63.246) (end 120.904 64.516) (width 0.25) (layer B.Cu) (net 4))
 (segment (start 106.426 63.246) (end 119.634 63.246) (width 0.25) (layer B.Cu) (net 4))
 (segment (start 108.761499 67.938) (end 105.918 65.094501) (width 0.25) (layer B.Cu) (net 4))
 (segment (start 111.506 67.938) (end 108.761499 67.938) (width 0.25) (layer B.Cu) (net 4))
 (segment (start 112.95 71.882) (end 111.506 70.438) (width 0.25) (layer B.Cu) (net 8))
 (segment (start 115.824 71.882) (end 112.95 71.882) (width 0.25) (layer B.Cu) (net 8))
 (segment (start 118.618 81.788) (end 123.444 76.962) (width 0.25) (layer B.Cu) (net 6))
 (segment (start 110.236 81.788) (end 118.618 81.788) (width 0.25) (layer B.Cu) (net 6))
 (segment (start 109.80701 81.35901) (end 110.236 81.788) (width 0.25) (layer B.Cu) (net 6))
 (segment (start 109.80701 79.63699) (end 109.80701 81.35901) (width 0.25) (layer B.Cu) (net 6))
 (segment (start 111.506 77.938) (end 109.80701 79.63699) (width 0.25) (layer B.Cu) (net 6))
 (segment (start 115.824 83.82) (end 121.412 83.82) (width 0.25) (layer B.Cu) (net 6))
 (segment (start 121.412 83.82) (end 124.714 80.518) (width 0.25) (layer B.Cu) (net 6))
 (segment (start 124.714 78.232) (end 123.444 76.962) (width 0.25) (layer B.Cu) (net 6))
 (segment (start 124.714 80.518) (end 124.714 78.232) (width 0.25) (layer B.Cu) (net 6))
 (segment (start 116.84 81.026) (end 123.444 74.422) (width 0.25) (layer B.Cu) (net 5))
 (segment (start 112.094 81.026) (end 116.84 81.026) (width 0.25) (layer B.Cu) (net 5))
 (segment (start 111.506 80.438) (end 112.094 81.026) (width 0.25) (layer B.Cu) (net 5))
 (segment (start 125.222 76.2) (end 123.444 74.422) (width 0.25) (layer B.Cu) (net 5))
 (segment (start 125.222 82.042) (end 125.222 76.2) (width 0.25) (layer B.Cu) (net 5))
 (segment (start 123.444 83.82) (end 125.222 82.042) (width 0.25) (layer B.Cu) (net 5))
 (segment (start 120.65 82.296) (end 123.444 79.502) (width 0.25) (layer B.Cu) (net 7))
 (segment (start 107.188 72.136) (end 107.188 74.422) (width 0.25) (layer B.Cu) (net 7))
 (segment (start 107.188 79.756) (end 109.728 82.296) (width 0.25) (layer B.Cu) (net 7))
 (segment (start 107.188 74.422) (end 107.188 79.756) (width 0.25) (layer B.Cu) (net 7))
 (segment (start 109.728 82.296) (end 120.65 82.296) (width 0.25) (layer B.Cu) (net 7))
 (segment (start 123.444 71.882) (end 123.444 68.326) (width 0.25) (layer B.Cu) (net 3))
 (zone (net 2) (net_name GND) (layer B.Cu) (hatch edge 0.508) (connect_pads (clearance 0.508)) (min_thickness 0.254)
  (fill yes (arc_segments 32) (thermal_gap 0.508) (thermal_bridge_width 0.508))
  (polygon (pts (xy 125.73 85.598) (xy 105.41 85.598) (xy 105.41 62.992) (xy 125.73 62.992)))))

